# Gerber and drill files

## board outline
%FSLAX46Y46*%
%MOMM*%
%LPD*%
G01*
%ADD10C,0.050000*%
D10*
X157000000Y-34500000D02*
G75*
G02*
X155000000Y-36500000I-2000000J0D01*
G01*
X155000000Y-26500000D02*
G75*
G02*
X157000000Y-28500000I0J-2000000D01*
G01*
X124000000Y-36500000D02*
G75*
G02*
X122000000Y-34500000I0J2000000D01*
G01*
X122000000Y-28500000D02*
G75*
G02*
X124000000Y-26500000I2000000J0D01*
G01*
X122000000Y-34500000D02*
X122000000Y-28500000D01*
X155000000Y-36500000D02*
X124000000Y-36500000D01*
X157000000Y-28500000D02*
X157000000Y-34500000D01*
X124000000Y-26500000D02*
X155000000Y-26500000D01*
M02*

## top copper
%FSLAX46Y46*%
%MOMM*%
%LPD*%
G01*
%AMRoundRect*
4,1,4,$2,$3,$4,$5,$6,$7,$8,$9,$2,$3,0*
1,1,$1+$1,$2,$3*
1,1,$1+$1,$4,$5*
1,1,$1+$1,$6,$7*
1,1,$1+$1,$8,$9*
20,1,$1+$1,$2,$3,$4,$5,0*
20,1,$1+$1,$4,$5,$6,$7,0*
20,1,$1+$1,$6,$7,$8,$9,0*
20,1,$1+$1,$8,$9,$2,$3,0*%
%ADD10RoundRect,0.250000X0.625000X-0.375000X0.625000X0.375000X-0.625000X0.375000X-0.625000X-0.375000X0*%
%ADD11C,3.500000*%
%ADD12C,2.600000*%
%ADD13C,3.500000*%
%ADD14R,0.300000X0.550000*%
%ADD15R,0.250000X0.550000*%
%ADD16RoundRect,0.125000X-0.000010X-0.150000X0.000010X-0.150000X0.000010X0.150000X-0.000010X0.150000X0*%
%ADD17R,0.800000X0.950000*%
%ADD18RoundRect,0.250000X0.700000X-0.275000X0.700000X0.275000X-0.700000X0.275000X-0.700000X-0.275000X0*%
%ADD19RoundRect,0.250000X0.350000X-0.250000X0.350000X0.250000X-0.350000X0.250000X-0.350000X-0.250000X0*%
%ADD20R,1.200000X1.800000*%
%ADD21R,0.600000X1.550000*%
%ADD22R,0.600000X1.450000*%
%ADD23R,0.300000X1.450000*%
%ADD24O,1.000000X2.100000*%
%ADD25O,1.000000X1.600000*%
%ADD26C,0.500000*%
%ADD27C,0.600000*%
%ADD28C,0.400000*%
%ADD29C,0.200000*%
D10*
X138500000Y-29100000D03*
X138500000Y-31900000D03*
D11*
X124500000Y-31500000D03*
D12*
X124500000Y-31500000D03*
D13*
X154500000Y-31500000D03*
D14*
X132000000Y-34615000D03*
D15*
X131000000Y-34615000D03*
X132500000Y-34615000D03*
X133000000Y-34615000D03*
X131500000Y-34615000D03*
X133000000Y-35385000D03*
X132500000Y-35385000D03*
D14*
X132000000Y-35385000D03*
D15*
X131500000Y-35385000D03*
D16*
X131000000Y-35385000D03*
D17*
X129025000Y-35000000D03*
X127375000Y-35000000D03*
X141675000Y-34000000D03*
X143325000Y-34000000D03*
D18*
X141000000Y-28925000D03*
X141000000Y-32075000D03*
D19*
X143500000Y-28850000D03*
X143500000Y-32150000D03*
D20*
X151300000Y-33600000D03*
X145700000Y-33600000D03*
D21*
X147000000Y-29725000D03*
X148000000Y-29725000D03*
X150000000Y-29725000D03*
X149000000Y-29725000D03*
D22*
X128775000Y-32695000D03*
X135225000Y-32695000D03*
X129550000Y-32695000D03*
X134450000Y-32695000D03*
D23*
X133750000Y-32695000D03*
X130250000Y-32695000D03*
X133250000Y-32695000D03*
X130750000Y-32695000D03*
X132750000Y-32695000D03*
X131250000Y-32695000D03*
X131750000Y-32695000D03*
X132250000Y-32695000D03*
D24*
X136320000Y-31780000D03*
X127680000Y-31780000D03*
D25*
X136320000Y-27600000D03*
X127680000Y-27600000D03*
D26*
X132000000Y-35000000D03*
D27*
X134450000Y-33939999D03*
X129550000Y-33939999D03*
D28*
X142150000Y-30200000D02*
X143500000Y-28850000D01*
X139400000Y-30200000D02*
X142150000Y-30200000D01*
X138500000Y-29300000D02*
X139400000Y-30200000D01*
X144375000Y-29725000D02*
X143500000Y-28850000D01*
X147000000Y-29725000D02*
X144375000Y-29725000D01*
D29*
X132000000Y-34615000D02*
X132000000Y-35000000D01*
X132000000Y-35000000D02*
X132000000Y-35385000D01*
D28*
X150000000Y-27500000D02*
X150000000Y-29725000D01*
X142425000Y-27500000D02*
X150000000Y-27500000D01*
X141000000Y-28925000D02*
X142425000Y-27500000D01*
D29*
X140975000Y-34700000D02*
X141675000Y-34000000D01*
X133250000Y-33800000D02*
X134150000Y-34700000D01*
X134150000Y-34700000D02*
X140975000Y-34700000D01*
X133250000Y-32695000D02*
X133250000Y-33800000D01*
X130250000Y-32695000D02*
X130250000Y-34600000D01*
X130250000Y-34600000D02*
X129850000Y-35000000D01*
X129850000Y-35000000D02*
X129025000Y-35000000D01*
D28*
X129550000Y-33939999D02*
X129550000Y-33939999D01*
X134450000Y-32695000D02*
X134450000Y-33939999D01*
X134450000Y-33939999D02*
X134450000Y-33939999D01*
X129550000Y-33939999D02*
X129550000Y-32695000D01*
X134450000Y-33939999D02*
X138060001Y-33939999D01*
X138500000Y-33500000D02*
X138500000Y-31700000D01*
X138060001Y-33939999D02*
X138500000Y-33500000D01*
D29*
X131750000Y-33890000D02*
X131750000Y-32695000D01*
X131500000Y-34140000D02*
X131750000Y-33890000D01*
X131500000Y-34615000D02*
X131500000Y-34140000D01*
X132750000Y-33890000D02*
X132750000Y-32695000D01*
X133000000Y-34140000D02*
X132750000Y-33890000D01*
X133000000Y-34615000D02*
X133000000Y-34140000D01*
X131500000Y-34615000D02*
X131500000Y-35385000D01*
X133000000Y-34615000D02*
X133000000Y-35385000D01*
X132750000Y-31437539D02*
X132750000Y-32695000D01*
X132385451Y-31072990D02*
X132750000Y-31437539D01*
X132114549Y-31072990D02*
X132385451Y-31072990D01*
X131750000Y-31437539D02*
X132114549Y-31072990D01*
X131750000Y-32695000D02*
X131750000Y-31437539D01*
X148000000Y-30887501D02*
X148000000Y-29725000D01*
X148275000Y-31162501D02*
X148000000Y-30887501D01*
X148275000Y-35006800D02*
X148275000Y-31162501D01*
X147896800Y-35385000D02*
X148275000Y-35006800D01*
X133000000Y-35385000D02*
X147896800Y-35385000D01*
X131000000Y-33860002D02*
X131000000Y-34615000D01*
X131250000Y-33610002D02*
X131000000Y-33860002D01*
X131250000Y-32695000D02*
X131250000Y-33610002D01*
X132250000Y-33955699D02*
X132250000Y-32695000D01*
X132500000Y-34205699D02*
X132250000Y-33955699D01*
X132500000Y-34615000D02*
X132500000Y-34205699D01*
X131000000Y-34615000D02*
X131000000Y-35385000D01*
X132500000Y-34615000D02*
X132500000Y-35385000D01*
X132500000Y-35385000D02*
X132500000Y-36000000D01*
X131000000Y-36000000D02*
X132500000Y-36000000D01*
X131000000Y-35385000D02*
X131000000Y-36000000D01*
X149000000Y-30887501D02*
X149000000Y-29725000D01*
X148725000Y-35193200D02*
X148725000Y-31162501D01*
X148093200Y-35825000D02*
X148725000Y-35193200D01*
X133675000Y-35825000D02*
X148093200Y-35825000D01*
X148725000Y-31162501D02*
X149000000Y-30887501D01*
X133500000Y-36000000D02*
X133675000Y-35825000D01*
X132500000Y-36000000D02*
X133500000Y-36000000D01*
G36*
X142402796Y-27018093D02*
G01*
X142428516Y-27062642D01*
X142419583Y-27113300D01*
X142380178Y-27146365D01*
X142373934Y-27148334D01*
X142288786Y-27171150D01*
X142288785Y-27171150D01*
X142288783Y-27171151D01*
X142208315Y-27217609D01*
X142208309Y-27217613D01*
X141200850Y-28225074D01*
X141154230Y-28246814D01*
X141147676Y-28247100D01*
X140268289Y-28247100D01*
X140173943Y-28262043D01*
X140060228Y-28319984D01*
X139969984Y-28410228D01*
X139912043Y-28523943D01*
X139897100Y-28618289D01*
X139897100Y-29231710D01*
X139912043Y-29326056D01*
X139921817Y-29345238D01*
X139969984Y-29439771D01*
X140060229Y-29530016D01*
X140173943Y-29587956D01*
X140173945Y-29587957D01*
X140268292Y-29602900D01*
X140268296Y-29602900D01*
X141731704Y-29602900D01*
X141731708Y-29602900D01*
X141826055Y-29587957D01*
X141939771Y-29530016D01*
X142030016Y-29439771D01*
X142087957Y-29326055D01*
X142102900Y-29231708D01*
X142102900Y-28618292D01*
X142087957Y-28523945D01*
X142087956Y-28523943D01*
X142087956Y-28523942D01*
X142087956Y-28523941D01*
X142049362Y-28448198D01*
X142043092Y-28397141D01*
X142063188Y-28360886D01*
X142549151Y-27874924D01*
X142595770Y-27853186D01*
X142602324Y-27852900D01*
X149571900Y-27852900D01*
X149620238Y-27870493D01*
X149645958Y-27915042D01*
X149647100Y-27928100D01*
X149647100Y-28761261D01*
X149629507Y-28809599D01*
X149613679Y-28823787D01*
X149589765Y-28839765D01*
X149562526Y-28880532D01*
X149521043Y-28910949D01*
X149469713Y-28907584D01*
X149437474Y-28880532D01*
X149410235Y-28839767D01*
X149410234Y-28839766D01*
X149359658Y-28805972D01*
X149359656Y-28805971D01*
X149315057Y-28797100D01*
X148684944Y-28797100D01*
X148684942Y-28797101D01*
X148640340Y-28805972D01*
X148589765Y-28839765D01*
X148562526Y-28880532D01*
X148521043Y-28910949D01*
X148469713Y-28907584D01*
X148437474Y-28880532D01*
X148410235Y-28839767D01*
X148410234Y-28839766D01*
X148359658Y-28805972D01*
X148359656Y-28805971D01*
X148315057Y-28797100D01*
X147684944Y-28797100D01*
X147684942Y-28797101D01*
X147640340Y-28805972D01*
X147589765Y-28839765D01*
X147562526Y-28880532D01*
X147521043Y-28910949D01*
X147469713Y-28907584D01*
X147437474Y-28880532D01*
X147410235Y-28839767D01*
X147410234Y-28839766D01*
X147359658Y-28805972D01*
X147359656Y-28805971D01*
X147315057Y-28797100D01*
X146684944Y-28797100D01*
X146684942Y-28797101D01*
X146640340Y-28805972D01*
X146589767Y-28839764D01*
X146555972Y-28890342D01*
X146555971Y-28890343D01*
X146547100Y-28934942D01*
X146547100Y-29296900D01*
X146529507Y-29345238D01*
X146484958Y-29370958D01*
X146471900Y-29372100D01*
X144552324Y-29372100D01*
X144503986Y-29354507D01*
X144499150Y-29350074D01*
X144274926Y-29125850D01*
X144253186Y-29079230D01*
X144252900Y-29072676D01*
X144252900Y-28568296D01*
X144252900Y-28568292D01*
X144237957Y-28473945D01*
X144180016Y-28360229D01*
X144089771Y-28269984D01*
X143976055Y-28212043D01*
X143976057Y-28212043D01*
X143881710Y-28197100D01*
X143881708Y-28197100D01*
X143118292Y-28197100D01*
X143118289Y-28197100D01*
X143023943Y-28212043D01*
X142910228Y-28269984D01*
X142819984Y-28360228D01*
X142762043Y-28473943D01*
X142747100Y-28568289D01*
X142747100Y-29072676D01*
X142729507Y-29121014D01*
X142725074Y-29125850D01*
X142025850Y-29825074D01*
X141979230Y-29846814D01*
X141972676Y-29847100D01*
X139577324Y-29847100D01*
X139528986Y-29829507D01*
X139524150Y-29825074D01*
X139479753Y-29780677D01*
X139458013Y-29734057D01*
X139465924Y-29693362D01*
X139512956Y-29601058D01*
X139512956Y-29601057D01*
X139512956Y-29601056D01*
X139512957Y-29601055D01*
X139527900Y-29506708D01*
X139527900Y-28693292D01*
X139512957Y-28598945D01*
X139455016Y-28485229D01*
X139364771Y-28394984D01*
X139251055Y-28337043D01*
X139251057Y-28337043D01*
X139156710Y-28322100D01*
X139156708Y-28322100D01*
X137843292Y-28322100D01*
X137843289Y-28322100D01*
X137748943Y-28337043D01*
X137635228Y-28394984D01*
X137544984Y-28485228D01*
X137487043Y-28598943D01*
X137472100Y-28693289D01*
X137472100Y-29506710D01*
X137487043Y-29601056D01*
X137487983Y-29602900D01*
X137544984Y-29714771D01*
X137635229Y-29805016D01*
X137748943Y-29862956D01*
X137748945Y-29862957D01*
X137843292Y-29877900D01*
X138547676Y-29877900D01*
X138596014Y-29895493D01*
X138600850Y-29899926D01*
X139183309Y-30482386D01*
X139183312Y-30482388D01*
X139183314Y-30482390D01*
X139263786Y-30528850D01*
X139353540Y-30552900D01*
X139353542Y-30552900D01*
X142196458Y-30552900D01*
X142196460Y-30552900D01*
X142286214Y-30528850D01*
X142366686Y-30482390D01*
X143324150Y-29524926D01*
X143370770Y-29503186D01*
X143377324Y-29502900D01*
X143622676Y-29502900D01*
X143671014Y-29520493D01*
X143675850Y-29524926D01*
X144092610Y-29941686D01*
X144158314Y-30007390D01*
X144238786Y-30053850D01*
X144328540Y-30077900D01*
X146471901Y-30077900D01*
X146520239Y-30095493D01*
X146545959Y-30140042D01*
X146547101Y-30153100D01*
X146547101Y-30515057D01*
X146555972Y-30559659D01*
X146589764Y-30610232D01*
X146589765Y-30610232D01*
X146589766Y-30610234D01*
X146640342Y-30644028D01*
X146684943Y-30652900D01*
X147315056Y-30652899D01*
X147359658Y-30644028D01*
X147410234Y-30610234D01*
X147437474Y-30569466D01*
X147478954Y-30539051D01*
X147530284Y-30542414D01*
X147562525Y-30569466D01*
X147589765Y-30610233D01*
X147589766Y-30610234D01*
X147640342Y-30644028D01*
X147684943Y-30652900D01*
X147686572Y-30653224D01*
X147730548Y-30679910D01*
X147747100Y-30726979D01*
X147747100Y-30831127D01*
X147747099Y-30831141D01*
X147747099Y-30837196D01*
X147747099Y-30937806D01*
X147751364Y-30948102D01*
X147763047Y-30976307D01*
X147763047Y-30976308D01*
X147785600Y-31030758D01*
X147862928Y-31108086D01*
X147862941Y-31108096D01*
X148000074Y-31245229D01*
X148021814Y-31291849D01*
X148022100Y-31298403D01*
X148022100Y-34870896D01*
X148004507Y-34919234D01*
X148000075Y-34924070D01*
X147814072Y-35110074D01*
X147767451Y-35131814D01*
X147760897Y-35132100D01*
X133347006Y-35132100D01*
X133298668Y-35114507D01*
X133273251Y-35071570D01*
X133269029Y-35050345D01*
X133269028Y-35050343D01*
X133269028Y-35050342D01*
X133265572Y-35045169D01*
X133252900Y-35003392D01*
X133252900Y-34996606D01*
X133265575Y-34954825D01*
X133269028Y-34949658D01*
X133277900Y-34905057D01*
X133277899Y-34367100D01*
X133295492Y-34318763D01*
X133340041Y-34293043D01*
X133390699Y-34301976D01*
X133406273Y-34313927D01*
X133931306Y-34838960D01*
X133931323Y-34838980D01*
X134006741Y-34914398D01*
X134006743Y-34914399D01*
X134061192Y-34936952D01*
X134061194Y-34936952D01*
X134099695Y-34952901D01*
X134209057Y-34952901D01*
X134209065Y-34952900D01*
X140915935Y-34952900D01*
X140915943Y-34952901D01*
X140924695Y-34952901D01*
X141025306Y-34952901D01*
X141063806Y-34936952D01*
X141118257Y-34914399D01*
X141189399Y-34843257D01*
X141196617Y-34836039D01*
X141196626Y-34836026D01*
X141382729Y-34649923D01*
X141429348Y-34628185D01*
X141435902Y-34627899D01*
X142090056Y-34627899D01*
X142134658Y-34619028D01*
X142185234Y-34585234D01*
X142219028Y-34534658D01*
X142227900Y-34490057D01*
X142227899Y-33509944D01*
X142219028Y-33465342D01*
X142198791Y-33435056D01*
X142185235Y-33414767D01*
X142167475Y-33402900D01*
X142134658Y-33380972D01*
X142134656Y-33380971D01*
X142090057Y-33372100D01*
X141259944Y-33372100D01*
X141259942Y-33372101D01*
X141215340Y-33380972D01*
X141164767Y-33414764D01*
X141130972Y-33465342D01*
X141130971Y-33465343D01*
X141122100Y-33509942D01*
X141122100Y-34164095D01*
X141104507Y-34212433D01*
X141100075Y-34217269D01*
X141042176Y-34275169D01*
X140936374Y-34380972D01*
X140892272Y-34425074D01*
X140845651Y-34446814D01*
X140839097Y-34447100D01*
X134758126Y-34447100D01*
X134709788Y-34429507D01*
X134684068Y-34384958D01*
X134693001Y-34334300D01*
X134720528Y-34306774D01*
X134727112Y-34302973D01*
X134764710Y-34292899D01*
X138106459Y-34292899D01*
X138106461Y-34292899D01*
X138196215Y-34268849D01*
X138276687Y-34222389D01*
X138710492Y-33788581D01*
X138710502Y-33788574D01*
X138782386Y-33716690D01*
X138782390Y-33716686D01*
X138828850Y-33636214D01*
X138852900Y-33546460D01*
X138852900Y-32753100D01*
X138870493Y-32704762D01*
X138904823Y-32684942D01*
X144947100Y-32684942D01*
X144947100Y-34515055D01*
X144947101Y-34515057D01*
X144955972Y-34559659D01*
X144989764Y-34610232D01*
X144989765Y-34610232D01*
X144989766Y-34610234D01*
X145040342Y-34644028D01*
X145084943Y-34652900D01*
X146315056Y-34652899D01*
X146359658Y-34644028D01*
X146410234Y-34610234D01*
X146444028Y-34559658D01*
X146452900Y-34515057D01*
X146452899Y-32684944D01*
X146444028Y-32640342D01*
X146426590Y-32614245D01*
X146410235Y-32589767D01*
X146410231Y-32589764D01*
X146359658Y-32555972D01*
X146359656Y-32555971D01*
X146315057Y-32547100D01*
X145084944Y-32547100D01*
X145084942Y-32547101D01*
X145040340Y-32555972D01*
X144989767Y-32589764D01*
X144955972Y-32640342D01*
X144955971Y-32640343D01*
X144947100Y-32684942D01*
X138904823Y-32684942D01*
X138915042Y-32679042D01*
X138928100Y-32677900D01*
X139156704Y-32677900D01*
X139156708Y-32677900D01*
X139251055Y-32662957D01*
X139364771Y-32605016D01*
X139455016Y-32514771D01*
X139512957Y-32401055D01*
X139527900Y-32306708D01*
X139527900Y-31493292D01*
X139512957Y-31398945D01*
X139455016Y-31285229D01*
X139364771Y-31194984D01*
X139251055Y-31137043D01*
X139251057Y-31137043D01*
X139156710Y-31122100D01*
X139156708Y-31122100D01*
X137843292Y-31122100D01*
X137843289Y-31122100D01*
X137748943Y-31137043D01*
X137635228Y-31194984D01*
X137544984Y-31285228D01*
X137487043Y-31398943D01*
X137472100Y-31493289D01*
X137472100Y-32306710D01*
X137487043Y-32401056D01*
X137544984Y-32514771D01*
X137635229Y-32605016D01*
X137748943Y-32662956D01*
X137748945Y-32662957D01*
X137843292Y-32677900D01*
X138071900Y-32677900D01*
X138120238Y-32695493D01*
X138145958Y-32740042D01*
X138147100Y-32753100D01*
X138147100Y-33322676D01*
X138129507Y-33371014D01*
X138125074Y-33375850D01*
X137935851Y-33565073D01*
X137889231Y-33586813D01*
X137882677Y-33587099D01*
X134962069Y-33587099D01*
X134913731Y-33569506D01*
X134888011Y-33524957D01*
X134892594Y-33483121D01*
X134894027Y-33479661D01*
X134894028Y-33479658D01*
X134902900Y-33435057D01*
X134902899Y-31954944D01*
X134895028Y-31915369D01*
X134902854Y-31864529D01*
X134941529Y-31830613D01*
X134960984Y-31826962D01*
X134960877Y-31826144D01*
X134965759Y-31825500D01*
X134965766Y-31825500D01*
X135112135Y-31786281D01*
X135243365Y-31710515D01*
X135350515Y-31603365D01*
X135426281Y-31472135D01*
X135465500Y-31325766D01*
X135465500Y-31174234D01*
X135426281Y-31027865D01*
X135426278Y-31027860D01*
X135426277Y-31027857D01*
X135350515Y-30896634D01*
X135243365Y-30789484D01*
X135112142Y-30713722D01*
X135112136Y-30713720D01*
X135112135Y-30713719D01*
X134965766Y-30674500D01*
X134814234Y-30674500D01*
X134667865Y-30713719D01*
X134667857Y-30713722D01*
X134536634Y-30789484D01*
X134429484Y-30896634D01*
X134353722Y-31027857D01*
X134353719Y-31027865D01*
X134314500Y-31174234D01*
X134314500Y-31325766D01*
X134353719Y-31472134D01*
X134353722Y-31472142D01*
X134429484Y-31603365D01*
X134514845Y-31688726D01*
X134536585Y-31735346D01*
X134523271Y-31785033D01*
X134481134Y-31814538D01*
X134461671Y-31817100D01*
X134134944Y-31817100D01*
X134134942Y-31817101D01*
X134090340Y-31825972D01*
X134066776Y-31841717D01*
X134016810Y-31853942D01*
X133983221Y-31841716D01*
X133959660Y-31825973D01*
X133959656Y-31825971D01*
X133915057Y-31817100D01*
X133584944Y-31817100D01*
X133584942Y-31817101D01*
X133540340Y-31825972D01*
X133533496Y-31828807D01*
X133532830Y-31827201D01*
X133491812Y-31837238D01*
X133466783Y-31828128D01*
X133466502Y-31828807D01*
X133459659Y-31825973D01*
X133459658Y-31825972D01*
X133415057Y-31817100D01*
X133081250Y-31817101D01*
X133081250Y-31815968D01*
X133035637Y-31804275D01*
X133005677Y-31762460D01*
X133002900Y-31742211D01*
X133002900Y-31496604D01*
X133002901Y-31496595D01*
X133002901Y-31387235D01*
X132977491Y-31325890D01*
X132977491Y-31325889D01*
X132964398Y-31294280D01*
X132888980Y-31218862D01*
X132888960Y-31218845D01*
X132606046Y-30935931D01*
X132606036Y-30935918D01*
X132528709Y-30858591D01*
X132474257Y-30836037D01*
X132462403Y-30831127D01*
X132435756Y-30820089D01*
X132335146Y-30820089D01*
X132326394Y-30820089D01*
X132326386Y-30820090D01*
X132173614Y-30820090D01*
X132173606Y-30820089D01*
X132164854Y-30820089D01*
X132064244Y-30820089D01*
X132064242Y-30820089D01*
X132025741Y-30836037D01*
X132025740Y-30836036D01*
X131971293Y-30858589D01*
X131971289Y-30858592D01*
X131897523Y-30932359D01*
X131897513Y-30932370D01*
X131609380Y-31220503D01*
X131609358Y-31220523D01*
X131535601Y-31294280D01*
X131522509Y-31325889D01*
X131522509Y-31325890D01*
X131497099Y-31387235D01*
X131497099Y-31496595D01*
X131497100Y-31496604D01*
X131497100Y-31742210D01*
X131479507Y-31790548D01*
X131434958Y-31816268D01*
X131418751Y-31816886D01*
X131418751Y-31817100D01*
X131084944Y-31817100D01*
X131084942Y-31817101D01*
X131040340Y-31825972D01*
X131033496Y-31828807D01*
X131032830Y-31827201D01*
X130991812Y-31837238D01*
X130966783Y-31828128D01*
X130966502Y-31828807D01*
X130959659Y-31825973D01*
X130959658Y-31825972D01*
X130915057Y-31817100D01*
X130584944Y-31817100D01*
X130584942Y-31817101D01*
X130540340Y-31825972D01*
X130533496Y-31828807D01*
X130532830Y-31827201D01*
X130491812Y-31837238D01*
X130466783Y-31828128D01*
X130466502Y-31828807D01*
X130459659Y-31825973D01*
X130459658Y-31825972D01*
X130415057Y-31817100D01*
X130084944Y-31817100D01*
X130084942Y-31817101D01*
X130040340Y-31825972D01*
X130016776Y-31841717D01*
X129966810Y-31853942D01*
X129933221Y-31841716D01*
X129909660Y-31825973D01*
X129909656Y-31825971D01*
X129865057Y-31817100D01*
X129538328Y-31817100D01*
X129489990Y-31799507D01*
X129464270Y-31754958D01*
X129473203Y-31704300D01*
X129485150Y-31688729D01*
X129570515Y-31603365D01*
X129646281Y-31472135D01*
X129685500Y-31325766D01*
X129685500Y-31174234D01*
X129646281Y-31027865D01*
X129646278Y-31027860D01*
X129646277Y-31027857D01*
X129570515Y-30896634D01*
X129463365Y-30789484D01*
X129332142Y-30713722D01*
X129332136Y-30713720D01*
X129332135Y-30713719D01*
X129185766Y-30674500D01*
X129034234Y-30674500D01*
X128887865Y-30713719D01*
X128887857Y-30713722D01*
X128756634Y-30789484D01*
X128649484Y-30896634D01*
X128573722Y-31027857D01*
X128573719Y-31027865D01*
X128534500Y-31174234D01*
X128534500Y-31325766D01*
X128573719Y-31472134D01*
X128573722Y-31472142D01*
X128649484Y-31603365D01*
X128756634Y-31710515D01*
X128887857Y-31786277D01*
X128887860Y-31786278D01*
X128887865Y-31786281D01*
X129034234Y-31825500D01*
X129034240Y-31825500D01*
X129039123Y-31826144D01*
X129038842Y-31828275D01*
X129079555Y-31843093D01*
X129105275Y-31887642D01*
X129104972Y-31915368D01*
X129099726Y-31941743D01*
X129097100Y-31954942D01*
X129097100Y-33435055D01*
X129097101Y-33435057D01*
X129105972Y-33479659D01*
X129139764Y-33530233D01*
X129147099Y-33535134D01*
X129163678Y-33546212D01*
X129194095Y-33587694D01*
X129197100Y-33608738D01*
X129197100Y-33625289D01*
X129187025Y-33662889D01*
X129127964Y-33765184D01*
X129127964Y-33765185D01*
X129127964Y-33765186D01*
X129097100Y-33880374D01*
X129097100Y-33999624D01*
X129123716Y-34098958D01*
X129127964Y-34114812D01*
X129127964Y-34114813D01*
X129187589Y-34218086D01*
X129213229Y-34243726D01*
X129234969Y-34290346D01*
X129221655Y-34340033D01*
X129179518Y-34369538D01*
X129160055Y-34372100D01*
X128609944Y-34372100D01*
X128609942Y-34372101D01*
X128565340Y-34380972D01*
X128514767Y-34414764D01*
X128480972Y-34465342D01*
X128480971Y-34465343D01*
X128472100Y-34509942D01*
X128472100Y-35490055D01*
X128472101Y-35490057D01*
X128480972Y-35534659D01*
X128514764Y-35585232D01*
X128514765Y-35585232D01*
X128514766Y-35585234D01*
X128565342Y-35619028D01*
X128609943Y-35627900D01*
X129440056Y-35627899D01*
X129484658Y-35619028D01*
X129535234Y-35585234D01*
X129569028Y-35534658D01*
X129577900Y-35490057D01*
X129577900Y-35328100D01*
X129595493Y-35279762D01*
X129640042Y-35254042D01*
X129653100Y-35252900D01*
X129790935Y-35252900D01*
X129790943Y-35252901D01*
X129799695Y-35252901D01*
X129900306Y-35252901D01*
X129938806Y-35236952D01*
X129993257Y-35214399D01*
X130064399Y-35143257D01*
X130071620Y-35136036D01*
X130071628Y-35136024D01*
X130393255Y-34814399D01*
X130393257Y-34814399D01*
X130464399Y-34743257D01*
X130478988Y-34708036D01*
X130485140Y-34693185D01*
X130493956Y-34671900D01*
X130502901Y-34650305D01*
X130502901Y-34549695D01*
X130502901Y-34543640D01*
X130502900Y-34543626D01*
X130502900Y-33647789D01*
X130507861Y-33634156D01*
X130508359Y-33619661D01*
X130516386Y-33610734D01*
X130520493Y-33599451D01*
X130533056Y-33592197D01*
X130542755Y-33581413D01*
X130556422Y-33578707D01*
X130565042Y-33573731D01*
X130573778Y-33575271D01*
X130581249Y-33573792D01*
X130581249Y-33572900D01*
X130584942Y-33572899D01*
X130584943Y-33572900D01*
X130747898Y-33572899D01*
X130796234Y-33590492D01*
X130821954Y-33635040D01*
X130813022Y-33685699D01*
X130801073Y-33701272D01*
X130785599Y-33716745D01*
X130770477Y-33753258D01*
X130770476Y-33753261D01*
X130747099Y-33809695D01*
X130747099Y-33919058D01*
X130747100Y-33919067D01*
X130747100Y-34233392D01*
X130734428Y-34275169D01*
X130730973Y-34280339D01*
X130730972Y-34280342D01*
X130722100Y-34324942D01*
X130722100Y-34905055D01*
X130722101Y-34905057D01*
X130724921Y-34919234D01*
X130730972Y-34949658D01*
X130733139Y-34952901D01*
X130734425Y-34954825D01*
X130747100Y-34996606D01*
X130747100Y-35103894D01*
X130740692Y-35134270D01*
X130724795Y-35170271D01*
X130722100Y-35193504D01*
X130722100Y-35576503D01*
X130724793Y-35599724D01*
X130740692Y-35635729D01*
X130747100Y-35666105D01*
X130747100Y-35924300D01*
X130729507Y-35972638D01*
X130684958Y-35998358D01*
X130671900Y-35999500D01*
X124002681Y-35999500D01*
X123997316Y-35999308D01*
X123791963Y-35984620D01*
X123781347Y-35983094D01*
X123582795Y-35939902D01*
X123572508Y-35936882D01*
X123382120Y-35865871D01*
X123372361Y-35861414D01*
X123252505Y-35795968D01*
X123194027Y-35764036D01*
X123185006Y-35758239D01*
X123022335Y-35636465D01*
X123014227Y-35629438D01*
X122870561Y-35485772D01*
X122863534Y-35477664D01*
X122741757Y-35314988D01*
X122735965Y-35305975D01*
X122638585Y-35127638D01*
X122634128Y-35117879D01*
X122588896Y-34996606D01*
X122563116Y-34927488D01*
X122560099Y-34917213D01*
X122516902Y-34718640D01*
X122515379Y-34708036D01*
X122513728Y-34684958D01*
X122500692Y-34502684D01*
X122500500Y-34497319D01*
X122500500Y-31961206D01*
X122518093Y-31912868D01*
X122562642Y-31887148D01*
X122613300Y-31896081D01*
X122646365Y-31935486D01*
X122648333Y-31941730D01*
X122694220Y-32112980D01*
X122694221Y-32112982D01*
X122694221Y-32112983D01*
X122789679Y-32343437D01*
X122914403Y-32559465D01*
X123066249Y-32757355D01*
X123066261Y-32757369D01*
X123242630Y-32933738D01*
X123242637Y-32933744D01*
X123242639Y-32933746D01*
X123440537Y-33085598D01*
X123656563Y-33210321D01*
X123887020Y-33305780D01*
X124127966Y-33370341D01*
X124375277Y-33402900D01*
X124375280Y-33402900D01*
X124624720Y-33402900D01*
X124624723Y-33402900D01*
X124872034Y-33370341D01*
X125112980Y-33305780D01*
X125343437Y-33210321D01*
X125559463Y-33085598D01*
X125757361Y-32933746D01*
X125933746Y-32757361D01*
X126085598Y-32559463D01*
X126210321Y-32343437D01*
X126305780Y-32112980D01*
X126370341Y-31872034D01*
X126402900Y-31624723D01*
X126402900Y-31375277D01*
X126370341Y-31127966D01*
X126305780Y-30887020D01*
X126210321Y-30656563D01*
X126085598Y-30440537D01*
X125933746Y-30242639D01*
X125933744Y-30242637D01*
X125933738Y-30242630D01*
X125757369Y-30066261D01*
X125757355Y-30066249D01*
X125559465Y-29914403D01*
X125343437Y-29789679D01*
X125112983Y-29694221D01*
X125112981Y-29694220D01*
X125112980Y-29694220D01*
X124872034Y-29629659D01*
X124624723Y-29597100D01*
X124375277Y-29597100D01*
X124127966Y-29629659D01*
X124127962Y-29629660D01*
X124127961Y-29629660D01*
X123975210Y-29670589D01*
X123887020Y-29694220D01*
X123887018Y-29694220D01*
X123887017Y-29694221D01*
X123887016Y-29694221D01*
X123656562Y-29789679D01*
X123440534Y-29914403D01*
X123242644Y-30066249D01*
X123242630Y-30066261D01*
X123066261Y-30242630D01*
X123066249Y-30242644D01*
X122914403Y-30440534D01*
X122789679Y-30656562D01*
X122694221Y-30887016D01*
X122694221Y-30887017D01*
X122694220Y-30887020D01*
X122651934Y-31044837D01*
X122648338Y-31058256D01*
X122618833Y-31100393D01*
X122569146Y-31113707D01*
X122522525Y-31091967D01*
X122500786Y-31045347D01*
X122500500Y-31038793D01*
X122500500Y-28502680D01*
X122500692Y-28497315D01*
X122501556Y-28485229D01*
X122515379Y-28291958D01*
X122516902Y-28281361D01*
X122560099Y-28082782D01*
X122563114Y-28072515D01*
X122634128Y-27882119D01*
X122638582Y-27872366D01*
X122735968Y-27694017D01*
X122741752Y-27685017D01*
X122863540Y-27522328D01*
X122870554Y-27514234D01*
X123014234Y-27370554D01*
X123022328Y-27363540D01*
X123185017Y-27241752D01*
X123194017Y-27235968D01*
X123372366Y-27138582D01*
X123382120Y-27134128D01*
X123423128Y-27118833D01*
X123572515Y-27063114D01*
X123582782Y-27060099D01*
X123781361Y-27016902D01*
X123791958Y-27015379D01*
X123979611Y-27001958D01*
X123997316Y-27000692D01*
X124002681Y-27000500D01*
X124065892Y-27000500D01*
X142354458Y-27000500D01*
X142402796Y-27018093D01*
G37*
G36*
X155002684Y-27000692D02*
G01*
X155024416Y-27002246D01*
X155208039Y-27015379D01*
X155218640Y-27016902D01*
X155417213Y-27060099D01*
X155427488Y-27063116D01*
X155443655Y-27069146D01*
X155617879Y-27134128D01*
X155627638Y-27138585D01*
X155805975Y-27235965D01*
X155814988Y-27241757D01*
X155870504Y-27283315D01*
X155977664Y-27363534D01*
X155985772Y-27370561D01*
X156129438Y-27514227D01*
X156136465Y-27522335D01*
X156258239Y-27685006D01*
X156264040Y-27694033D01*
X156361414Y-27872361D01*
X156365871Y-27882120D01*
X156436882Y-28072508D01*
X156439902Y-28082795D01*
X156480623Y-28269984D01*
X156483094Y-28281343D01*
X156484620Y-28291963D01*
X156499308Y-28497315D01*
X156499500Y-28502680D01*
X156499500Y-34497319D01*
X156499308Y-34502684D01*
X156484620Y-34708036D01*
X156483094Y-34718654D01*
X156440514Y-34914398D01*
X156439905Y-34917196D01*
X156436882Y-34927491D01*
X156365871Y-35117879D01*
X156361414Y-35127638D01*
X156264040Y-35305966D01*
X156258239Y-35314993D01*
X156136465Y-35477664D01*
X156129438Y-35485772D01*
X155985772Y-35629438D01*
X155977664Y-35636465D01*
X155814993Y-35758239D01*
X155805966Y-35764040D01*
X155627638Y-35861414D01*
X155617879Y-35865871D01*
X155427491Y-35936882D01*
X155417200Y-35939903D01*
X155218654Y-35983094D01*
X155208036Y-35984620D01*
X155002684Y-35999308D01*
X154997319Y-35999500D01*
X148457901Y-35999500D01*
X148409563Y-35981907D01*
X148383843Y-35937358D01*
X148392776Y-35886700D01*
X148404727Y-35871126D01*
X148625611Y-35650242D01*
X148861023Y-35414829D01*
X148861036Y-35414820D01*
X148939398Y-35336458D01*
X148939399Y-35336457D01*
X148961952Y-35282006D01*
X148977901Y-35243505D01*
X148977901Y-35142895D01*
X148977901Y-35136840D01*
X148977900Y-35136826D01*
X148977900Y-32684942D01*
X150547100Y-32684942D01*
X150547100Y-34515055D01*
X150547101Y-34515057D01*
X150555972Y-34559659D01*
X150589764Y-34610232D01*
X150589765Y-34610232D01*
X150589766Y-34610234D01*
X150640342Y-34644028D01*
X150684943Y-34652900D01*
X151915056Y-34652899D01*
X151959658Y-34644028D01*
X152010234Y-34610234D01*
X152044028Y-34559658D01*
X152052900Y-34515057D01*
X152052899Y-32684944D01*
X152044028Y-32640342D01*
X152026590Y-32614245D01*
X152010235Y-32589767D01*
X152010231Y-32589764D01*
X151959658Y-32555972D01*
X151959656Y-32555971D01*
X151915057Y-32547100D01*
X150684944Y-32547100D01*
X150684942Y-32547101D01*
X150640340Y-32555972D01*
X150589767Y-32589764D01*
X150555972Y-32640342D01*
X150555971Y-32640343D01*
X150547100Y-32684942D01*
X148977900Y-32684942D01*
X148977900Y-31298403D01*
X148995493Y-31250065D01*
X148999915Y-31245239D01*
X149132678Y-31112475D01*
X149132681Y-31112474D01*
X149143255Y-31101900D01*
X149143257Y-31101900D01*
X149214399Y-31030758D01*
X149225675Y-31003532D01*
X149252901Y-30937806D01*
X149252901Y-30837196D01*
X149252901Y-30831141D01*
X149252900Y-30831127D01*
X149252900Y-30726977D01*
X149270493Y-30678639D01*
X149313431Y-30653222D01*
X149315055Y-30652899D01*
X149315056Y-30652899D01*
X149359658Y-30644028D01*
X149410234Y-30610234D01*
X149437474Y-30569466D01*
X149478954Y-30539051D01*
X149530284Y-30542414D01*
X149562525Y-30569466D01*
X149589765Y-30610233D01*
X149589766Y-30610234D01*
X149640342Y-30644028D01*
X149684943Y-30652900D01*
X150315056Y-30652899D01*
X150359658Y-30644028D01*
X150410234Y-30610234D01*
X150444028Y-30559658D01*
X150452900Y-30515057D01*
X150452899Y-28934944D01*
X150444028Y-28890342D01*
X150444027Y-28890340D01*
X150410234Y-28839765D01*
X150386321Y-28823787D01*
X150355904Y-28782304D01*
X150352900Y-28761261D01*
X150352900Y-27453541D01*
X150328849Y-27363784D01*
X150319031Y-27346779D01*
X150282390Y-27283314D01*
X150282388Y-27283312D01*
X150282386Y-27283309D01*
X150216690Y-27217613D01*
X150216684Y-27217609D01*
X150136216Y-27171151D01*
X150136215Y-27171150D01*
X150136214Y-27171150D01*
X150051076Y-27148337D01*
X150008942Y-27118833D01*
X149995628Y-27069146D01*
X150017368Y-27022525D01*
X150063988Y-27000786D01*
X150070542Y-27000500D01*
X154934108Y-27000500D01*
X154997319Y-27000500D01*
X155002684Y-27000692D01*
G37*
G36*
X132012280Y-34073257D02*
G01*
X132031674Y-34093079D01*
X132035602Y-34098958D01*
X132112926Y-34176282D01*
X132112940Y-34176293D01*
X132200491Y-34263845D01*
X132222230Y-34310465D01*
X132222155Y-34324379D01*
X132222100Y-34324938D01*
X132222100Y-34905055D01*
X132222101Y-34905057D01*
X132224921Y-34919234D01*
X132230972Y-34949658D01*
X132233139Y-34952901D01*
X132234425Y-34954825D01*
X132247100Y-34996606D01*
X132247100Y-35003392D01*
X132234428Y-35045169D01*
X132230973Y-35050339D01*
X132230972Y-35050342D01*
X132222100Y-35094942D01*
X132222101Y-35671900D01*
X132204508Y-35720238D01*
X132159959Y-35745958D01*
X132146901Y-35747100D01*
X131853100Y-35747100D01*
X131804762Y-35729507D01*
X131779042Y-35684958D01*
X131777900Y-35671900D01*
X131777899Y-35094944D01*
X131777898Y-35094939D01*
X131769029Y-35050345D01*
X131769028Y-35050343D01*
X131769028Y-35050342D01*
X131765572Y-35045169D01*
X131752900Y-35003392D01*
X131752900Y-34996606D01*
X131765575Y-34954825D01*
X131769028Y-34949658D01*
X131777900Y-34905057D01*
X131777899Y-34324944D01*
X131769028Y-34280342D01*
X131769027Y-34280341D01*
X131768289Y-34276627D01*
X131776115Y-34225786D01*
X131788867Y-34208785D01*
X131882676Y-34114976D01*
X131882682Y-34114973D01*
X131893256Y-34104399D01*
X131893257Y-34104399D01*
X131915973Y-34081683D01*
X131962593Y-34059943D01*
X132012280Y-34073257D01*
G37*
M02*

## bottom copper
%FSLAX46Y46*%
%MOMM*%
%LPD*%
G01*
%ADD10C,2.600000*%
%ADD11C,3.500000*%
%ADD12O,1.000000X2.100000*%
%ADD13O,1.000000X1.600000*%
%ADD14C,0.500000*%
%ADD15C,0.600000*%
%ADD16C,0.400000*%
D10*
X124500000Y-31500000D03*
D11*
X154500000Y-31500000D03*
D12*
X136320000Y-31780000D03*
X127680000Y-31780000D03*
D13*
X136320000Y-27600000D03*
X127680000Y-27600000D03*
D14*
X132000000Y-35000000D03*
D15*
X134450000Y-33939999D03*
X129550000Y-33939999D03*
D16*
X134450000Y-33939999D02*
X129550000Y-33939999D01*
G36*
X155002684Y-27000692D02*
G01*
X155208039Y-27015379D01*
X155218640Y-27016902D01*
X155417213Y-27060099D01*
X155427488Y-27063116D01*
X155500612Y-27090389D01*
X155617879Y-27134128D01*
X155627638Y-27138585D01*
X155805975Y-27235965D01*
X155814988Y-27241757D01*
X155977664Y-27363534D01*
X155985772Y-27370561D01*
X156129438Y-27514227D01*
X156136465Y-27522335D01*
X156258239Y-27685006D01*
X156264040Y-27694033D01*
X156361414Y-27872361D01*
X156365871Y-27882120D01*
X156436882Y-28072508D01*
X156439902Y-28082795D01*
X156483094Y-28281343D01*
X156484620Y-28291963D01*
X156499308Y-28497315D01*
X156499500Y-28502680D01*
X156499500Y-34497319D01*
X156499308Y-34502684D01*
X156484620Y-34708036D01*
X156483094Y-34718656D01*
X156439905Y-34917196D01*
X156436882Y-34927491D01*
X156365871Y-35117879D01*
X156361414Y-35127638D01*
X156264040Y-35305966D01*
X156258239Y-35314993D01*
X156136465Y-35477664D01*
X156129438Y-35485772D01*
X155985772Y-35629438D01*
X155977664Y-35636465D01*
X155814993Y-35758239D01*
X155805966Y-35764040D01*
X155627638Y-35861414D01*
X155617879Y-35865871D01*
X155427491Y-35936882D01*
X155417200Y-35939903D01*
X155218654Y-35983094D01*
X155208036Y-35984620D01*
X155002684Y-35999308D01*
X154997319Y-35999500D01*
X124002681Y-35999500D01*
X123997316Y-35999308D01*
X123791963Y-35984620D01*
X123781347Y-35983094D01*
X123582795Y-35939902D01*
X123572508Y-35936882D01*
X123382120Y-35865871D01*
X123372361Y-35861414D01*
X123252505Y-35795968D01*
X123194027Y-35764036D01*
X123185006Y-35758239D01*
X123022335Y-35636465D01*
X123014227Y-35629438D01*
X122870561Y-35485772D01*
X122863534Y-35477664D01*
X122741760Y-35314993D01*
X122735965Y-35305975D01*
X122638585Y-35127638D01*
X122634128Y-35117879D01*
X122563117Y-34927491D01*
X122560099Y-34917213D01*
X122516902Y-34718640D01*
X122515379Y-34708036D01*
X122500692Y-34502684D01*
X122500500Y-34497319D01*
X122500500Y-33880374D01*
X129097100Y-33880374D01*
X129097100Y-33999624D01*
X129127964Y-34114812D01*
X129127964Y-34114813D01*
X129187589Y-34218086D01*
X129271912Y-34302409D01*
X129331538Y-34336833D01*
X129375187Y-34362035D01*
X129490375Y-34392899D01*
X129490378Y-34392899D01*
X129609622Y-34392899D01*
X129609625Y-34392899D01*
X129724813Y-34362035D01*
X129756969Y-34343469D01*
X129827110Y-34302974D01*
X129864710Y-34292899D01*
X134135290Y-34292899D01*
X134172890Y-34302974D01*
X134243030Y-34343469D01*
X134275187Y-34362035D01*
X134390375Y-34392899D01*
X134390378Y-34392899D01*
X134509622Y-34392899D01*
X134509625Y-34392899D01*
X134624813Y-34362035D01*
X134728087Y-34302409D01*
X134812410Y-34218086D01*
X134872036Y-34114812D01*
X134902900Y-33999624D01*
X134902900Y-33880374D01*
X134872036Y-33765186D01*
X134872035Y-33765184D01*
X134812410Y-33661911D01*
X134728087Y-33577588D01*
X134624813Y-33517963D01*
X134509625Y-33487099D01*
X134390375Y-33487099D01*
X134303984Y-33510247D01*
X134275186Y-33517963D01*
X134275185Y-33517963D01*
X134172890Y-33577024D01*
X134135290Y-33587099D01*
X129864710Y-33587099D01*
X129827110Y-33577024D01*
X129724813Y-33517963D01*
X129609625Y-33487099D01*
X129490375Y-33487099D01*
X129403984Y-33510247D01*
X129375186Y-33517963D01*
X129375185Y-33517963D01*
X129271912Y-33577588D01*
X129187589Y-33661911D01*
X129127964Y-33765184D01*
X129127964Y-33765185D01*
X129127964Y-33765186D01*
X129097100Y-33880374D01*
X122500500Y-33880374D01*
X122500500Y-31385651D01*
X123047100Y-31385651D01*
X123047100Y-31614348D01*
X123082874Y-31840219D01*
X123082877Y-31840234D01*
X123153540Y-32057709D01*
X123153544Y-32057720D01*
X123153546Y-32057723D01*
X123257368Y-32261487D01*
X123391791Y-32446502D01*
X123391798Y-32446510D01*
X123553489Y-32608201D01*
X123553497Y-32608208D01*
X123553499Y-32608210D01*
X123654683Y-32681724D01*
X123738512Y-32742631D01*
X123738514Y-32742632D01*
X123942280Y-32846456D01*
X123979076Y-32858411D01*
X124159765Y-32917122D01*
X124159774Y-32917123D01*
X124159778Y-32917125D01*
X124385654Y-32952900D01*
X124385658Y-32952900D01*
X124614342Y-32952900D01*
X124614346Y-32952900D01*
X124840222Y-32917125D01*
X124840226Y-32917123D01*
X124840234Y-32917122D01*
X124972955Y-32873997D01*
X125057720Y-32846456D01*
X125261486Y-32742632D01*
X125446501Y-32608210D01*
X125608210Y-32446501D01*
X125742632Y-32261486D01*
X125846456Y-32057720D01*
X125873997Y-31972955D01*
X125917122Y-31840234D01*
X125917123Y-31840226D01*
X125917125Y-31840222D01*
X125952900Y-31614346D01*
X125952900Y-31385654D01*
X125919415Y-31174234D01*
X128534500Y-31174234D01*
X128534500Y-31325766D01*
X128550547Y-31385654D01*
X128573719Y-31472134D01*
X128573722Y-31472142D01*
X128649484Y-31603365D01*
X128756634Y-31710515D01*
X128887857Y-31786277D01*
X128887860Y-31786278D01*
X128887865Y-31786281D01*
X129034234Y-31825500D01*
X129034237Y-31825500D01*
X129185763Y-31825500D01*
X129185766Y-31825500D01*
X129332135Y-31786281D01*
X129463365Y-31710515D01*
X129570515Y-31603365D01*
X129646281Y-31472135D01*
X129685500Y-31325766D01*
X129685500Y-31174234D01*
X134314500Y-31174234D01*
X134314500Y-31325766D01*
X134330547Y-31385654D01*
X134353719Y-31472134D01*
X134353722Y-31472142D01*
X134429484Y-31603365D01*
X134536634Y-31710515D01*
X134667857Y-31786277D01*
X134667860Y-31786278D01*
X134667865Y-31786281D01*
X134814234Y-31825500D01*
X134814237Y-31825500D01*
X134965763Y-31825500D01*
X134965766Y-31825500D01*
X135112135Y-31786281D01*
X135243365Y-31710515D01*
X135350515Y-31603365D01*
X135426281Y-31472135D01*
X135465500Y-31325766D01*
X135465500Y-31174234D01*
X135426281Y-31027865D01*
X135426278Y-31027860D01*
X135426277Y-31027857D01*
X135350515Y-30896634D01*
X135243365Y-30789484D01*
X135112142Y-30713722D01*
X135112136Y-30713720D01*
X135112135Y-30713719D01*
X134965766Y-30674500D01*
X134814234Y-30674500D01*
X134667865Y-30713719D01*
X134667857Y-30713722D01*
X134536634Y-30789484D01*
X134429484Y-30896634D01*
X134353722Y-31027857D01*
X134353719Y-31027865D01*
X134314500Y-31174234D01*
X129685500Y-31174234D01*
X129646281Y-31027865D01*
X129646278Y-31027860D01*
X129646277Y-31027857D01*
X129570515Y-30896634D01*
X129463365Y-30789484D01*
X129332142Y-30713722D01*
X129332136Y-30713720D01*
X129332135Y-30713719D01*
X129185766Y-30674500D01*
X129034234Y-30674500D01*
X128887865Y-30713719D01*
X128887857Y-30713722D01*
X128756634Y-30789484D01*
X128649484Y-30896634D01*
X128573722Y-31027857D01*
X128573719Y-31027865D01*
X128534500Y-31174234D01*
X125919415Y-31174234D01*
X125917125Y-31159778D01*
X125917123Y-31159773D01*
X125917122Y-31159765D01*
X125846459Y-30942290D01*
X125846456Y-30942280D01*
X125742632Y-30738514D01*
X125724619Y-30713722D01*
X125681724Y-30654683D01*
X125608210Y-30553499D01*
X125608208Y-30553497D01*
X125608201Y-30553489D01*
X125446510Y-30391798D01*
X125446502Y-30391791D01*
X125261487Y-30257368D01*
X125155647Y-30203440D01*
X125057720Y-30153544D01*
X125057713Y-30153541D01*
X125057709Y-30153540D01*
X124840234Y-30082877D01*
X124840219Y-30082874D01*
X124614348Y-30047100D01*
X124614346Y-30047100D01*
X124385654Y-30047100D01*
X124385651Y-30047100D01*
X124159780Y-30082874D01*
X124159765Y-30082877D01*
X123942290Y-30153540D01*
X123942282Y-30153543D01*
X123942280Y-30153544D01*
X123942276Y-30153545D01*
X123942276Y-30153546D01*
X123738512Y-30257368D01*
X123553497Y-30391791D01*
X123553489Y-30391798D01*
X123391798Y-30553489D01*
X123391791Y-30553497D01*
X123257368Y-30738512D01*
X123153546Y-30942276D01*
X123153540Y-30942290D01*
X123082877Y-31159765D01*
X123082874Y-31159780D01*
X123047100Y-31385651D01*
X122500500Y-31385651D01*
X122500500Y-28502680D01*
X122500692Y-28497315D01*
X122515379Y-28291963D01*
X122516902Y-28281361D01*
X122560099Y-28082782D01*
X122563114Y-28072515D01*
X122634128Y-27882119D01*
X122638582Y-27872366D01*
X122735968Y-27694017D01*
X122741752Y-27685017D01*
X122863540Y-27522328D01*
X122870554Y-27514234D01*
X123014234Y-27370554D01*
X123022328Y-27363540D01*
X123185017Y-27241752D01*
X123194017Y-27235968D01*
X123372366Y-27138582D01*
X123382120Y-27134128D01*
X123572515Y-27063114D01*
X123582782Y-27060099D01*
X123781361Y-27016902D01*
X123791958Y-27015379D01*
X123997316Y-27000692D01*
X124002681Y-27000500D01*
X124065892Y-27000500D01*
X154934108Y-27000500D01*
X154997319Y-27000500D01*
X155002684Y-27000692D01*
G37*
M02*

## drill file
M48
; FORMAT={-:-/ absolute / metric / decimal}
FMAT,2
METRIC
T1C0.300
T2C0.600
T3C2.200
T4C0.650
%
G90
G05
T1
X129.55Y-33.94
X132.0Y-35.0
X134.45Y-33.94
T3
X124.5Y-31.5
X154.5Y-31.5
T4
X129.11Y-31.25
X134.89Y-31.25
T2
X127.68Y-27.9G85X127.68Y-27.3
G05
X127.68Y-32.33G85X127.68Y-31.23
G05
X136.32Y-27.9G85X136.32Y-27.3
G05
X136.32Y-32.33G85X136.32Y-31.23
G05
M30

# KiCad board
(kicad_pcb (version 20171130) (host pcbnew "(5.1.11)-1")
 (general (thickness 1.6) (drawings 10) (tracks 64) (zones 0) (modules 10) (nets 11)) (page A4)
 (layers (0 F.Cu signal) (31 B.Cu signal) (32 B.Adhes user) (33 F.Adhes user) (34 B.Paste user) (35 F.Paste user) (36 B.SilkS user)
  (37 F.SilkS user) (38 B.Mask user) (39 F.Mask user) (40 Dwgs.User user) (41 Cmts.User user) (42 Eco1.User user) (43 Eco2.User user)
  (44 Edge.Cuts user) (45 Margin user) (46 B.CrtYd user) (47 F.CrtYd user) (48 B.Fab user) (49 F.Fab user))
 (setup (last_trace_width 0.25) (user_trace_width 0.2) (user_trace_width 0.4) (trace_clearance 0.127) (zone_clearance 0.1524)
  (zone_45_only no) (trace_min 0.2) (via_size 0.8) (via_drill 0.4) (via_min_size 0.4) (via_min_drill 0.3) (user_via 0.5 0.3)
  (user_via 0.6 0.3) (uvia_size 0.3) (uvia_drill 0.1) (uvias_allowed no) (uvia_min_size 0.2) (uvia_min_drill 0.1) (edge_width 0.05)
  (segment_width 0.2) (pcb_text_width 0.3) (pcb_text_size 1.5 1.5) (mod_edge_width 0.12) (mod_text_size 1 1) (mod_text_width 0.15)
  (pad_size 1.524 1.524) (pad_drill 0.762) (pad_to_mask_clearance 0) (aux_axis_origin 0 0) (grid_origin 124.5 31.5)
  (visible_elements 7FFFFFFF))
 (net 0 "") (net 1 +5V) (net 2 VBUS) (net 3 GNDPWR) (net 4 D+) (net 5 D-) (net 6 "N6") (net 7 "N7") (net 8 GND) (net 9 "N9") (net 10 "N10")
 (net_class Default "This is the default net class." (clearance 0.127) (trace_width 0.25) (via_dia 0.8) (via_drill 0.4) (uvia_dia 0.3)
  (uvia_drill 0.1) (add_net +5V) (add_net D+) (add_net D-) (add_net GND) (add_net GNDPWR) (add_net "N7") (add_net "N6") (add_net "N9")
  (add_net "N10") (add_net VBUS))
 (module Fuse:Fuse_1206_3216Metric (layer F.Cu) (at 138.5 30.5 90)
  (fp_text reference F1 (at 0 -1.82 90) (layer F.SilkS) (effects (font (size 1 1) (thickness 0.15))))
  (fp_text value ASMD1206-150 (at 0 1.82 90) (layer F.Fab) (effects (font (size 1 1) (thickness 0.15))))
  (pad 2 smd roundrect (at 1.4 0 90) (size 1.25 1.75) (layers F.Cu F.Paste F.Mask) (roundrect_rratio 0.2) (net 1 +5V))
  (pad 1 smd roundrect (at -1.4 0 90) (size 1.25 1.75) (layers F.Cu F.Paste F.Mask) (roundrect_rratio 0.2) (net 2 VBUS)))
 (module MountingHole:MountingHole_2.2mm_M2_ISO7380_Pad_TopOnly (layer F.Cu) (at 124.5 31.5)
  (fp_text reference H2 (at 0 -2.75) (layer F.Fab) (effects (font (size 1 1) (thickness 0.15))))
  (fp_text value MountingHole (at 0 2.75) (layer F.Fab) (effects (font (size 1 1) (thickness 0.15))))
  (pad 1 connect circle (at 0 0) (size 3.5 3.5) (layers F.Cu F.Mask))
  (pad 1 thru_hole circle (at 0 0) (size 2.6 2.6) (drill 2.2) (layers *.Cu *.Mask)))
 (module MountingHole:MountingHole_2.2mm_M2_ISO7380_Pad (layer F.Cu) (at 154.5 31.5)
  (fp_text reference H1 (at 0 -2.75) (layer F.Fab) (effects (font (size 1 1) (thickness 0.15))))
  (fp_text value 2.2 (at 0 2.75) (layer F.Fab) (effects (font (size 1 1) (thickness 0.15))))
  (pad 1 thru_hole circle (at 0 0) (size 3.5 3.5) (drill 2.2) (layers *.Cu *.Mask) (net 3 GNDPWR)))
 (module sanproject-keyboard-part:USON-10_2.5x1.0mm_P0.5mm (layer F.Cu) (at 132 35 90)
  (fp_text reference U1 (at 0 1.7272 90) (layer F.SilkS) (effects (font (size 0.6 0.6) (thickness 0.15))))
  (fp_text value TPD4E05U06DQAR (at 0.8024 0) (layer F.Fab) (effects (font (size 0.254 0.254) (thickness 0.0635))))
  (pad 8 smd rect (at 0.385 0) (size 0.3 0.55) (layers F.Cu F.Paste F.Mask) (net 3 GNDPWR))
  (pad 10 smd rect (at 0.385 -1) (size 0.25 0.55) (layers F.Cu F.Paste F.Mask) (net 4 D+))
  (pad 7 smd rect (at 0.385 0.5) (size 0.25 0.55) (layers F.Cu F.Paste F.Mask) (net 4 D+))
  (pad 6 smd rect (at 0.385 1) (size 0.25 0.55) (layers F.Cu F.Paste F.Mask) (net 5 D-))
  (pad 9 smd rect (at 0.385 -0.5) (size 0.25 0.55) (layers F.Cu F.Paste F.Mask) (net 5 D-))
  (pad 5 smd rect (at -0.385 1) (size 0.25 0.55) (layers F.Cu F.Paste F.Mask) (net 5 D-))
  (pad 4 smd rect (at -0.385 0.5) (size 0.25 0.55) (layers F.Cu F.Paste F.Mask) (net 4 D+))
  (pad 3 smd rect (at -0.385 0) (size 0.3 0.55) (layers F.Cu F.Paste F.Mask) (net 3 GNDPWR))
  (pad 2 smd rect (at -0.385 -0.5) (size 0.25 0.55) (layers F.Cu F.Paste F.Mask) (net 5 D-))
  (pad 1 smd roundrect (at -0.385 -1) (size 0.25 0.55) (layers F.Cu F.Paste F.Mask) (roundrect_rratio 0.5) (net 4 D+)))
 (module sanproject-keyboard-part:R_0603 (layer F.Cu) (at 128.2 35)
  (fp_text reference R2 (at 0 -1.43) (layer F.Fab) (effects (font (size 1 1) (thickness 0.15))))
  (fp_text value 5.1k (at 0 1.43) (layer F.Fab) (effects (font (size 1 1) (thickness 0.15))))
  (pad 2 smd rect (at 0.825 0) (size 0.8 0.95) (layers F.Cu F.Paste F.Mask) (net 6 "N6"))
  (pad 1 smd rect (at -0.825 0) (size 0.8 0.95) (layers F.Cu F.Paste F.Mask) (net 3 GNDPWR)))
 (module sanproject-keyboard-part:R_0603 (layer F.Cu) (at 142.5 34 180)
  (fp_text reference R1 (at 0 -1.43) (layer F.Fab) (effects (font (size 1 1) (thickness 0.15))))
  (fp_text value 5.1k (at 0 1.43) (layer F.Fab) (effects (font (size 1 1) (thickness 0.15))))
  (pad 2 smd rect (at 0.825 0 180) (size 0.8 0.95) (layers F.Cu F.Paste F.Mask) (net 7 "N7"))
  (pad 1 smd rect (at -0.825 0 180) (size 0.8 0.95) (layers F.Cu F.Paste F.Mask) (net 3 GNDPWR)))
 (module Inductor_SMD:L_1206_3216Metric (layer F.Cu) (at 141 30.5 90)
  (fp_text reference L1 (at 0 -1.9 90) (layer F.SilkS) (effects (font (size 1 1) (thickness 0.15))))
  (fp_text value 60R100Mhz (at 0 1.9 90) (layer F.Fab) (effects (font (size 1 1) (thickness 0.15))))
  (pad 2 smd roundrect (at 1.575 0 90) (size 1.05 1.9) (layers F.Cu F.Paste F.Mask) (roundrect_rratio 0.238095) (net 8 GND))
  (pad 1 smd roundrect (at -1.575 0 90) (size 1.05 1.9) (layers F.Cu F.Paste F.Mask) (roundrect_rratio 0.238095) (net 3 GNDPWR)))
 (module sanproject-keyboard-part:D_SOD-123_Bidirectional (layer F.Cu) (at 143.5 30.5 90)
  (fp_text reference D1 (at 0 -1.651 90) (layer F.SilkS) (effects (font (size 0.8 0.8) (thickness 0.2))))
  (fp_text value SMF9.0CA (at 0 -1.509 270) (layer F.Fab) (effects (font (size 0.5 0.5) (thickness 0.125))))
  (pad 2 smd roundrect (at 1.65 0 90) (size 1 1.2) (layers F.Cu F.Paste F.Mask) (roundrect_rratio 0.25) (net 1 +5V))
  (pad 1 smd roundrect (at -1.65 0 90) (size 1 1.2) (layers F.Cu F.Paste F.Mask) (roundrect_rratio 0.25) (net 3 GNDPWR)))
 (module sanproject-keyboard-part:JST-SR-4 (layer F.Cu) (at 148.5 34.5)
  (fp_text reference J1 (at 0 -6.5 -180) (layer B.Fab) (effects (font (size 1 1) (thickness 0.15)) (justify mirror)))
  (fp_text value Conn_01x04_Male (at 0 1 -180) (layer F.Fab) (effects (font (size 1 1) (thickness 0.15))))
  (pad "" smd rect (at 2.8 -0.9) (size 1.2 1.8) (layers F.Cu F.Paste F.Mask))
  (pad "" smd rect (at -2.8 -0.9) (size 1.2 1.8) (layers F.Cu F.Paste F.Mask))
  (pad 1 smd rect (at -1.5 -4.775) (size 0.6 1.55) (layers F.Cu F.Paste F.Mask) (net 1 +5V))
  (pad 2 smd rect (at -0.5 -4.775) (size 0.6 1.55) (layers F.Cu F.Paste F.Mask) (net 5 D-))
  (pad 4 smd rect (at 1.5 -4.775) (size 0.6 1.55) (layers F.Cu F.Paste F.Mask) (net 8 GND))
  (pad 3 smd rect (at 0.5 -4.775) (size 0.6 1.55) (layers F.Cu F.Paste F.Mask) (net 4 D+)))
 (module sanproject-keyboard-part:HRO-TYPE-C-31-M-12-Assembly (layer F.Cu) (at 132 25 180)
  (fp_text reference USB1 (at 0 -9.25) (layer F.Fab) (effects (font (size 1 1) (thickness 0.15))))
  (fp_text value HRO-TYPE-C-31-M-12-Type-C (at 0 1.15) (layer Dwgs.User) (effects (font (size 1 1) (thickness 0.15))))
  (pad 12 smd rect (at 3.225 -7.695 180) (size 0.6 1.45) (layers F.Cu F.Paste F.Mask) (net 3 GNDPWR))
  (pad 1 smd rect (at -3.225 -7.695 180) (size 0.6 1.45) (layers F.Cu F.Paste F.Mask) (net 3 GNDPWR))
  (pad 11 smd rect (at 2.45 -7.695 180) (size 0.6 1.45) (layers F.Cu F.Paste F.Mask) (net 2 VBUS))
  (pad 2 smd rect (at -2.45 -7.695 180) (size 0.6 1.45) (layers F.Cu F.Paste F.Mask) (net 2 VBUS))
  (pad 3 smd rect (at -1.75 -7.695 180) (size 0.3 1.45) (layers F.Cu F.Paste F.Mask) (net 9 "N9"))
  (pad 10 smd rect (at 1.75 -7.695 180) (size 0.3 1.45) (layers F.Cu F.Paste F.Mask) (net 6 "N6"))
  (pad 4 smd rect (at -1.25 -7.695 180) (size 0.3 1.45) (layers F.Cu F.Paste F.Mask) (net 7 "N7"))
  (pad 9 smd rect (at 1.25 -7.695 180) (size 0.3 1.45) (layers F.Cu F.Paste F.Mask) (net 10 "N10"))
  (pad 5 smd rect (at -0.75 -7.695 180) (size 0.3 1.45) (layers F.Cu F.Paste F.Mask) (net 5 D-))
  (pad 8 smd rect (at 0.75 -7.695 180) (size 0.3 1.45) (layers F.Cu F.Paste F.Mask) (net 4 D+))
  (pad 7 smd rect (at 0.25 -7.695 180) (size 0.3 1.45) (layers F.Cu F.Paste F.Mask) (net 5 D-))
  (pad 6 smd rect (at -0.25 -7.695 180) (size 0.3 1.45) (layers F.Cu F.Paste F.Mask) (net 4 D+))
  (pad "" np_thru_hole circle (at 2.89 -6.25 180) (size 0.65 0.65) (drill 0.65) (layers *.Cu *.Mask))
  (pad "" np_thru_hole circle (at -2.89 -6.25 180) (size 0.65 0.65) (drill 0.65) (layers *.Cu *.Mask))
  (pad 13 thru_hole oval (at -4.32 -6.78 180) (size 1 2.1) (drill oval 0.6 1.7) (layers *.Cu *.Mask F.Paste) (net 3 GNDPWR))
  (pad 13 thru_hole oval (at 4.32 -6.78 180) (size 1 2.1) (drill oval 0.6 1.7) (layers *.Cu *.Mask F.Paste) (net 3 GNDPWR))
  (pad 13 thru_hole oval (at -4.32 -2.6 180) (size 1 1.6) (drill oval 0.6 1.2) (layers *.Cu *.Mask F.Paste) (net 3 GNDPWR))
  (pad 13 thru_hole oval (at 4.32 -2.6 180) (size 1 1.6) (drill oval 0.6 1.2) (layers *.Cu *.Mask F.Paste) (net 3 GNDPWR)))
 (gr_arc (start 155 34.5) (end 155 36.5) (angle -90) (layer Edge.Cuts) (width 0.05))
 (gr_arc (start 155 28.5) (end 157 28.5) (angle -90) (layer Edge.Cuts) (width 0.05))
 (gr_arc (start 124 34.5) (end 122 34.5) (angle -90) (layer Edge.Cuts) (width 0.05))
 (gr_arc (start 124 28.5) (end 124 26.5) (angle -90) (layer Edge.Cuts) (width 0.05))
 (gr_line (start 122 34.5) (end 122 28.5) (layer Edge.Cuts) (width 0.05))
 (gr_line (start 155 36.5) (end 124 36.5) (layer Edge.Cuts) (width 0.05))
 (gr_line (start 157 28.5) (end 157 34.5) (layer Edge.Cuts) (width 0.05))
 (gr_line (start 124 26.5) (end 155 26.5) (layer Edge.Cuts) (width 0.05))
 (segment (start 142.15 30.2) (end 143.5 28.85) (width 0.4) (layer F.Cu) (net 1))
 (segment (start 139.4 30.2) (end 142.15 30.2) (width 0.4) (layer F.Cu) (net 1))
 (segment (start 138.5 29.3) (end 139.4 30.2) (width 0.4) (layer F.Cu) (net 1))
 (segment (start 144.375 29.725) (end 143.5 28.85) (width 0.4) (layer F.Cu) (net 1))
 (segment (start 147 29.725) (end 144.375 29.725) (width 0.4) (layer F.Cu) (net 1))
 (via (at 132 35) (size 0.5) (drill 0.3) (layers F.Cu B.Cu) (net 3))
 (segment (start 132 34.615) (end 132 35) (width 0.2) (layer F.Cu) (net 3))
 (segment (start 132 35) (end 132 35.385) (width 0.2) (layer F.Cu) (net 3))
 (segment (start 150 27.5) (end 150 29.725) (width 0.4) (layer F.Cu) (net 8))
 (segment (start 142.425 27.5) (end 150 27.5) (width 0.4) (layer F.Cu) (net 8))
 (segment (start 141 28.925) (end 142.425 27.5) (width 0.4) (layer F.Cu) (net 8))
 (segment (start 140.975 34.7) (end 141.675 34) (width 0.2) (layer F.Cu) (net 7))
 (segment (start 133.25 33.8) (end 134.15 34.7) (width 0.2) (layer F.Cu) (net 7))
 (segment (start 134.15 34.7) (end 140.975 34.7) (width 0.2) (layer F.Cu) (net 7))
 (segment (start 133.25 32.695) (end 133.25 33.8) (width 0.2) (layer F.Cu) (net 7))
 (segment (start 130.25 32.695) (end 130.25 34.6) (width 0.2) (layer F.Cu) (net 6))
 (segment (start 130.25 34.6) (end 129.85 35) (width 0.2) (layer F.Cu) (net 6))
 (segment (start 129.85 35) (end 129.025 35) (width 0.2) (layer F.Cu) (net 6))
 (segment (start 129.55 33.939999) (end 129.55 33.939999) (width 0.4) (layer F.Cu) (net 2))
 (segment (start 134.45 32.695) (end 134.45 33.939999) (width 0.4) (layer F.Cu) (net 2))
 (segment (start 134.45 33.939999) (end 134.45 33.939999) (width 0.4) (layer F.Cu) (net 2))
 (via (at 134.45 33.939999) (size 0.6) (drill 0.3) (layers F.Cu B.Cu) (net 2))
 (segment (start 129.55 33.939999) (end 129.55 32.695) (width 0.4) (layer F.Cu) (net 2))
 (via (at 129.55 33.939999) (size 0.6) (drill 0.3) (layers F.Cu B.Cu) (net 2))
 (segment (start 134.45 33.939999) (end 129.55 33.939999) (width 0.4) (layer B.Cu) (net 2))
 (segment (start 134.45 33.939999) (end 138.060001 33.939999) (width 0.4) (layer F.Cu) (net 2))
 (segment (start 138.5 33.5) (end 138.5 31.7) (width 0.4) (layer F.Cu) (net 2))
 (segment (start 138.060001 33.939999) (end 138.5 33.5) (width 0.4) (layer F.Cu) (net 2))
 (segment (start 131.75 33.89) (end 131.75 32.695) (width 0.2) (layer F.Cu) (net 5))
 (segment (start 131.5 34.14) (end 131.75 33.89) (width 0.2) (layer F.Cu) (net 5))
 (segment (start 131.5 34.615) (end 131.5 34.14) (width 0.2) (layer F.Cu) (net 5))
 (segment (start 132.75 33.89) (end 132.75 32.695) (width 0.2) (layer F.Cu) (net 5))
 (segment (start 133 34.14) (end 132.75 33.89) (width 0.2) (layer F.Cu) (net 5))
 (segment (start 133 34.615) (end 133 34.14) (width 0.2) (layer F.Cu) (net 5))
 (segment (start 131.5 34.615) (end 131.5 35.385) (width 0.2) (layer F.Cu) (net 5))
 (segment (start 133 34.615) (end 133 35.385) (width 0.2) (layer F.Cu) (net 5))
 (segment (start 132.75 31.437539) (end 132.75 32.695) (width 0.2) (layer F.Cu) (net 5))
 (segment (start 132.385451 31.07299) (end 132.75 31.437539) (width 0.2) (layer F.Cu) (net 5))
 (segment (start 132.114549 31.07299) (end 132.385451 31.07299) (width 0.2) (layer F.Cu) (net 5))
 (segment (start 131.75 31.437539) (end 132.114549 31.07299) (width 0.2) (layer F.Cu) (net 5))
 (segment (start 131.75 32.695) (end 131.75 31.437539) (width 0.2) (layer F.Cu) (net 5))
 (segment (start 148 30.887501) (end 148 29.725) (width 0.2) (layer F.Cu) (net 5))
 (segment (start 148.275 31.162501) (end 148 30.887501) (width 0.2) (layer F.Cu) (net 5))
 (segment (start 148.275 35.0068) (end 148.275 31.162501) (width 0.2) (layer F.Cu) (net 5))
 (segment (start 147.8968 35.385) (end 148.275 35.0068) (width 0.2) (layer F.Cu) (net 5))
 (segment (start 133 35.385) (end 147.8968 35.385) (width 0.2) (layer F.Cu) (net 5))
 (segment (start 131 33.860002) (end 131 34.615) (width 0.2) (layer F.Cu) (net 4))
 (segment (start 131.25 33.610002) (end 131 33.860002) (width 0.2) (layer F.Cu) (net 4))
 (segment (start 131.25 32.695) (end 131.25 33.610002) (width 0.2) (layer F.Cu) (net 4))
 (segment (start 132.25 33.955699) (end 132.25 32.695) (width 0.2) (layer F.Cu) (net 4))
 (segment (start 132.5 34.205699) (end 132.25 33.955699) (width 0.2) (layer F.Cu) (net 4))
 (segment (start 132.5 34.615) (end 132.5 34.205699) (width 0.2) (layer F.Cu) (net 4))
 (segment (start 131 34.615) (end 131 35.385) (width 0.2) (layer F.Cu) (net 4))
 (segment (start 132.5 34.615) (end 132.5 35.385) (width 0.2) (layer F.Cu) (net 4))
 (segment (start 132.5 35.385) (end 132.5 36) (width 0.2) (layer F.Cu) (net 4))
 (segment (start 131 36) (end 132.5 36) (width 0.2) (layer F.Cu) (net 4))
 (segment (start 131 35.385) (end 131 36) (width 0.2) (layer F.Cu) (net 4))
 (segment (start 149 30.887501) (end 149 29.725) (width 0.2) (layer F.Cu) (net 4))
 (segment (start 148.725 35.1932) (end 148.725 31.162501) (width 0.2) (layer F.Cu) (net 4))
 (segment (start 148.0932 35.825) (end 148.725 35.1932) (width 0.2) (layer F.Cu) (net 4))
 (segment (start 133.675 35.825) (end 148.0932 35.825) (width 0.2) (layer F.Cu) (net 4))
 (segment (start 148.725 31.162501) (end 149 30.887501) (width 0.2) (layer F.Cu) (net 4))
 (segment (start 133.5 36) (end 133.675 35.825) (width 0.2) (layer F.Cu) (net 4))
 (segment (start 132.5 36) (end 133.5 36) (width 0.2) (layer F.Cu) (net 4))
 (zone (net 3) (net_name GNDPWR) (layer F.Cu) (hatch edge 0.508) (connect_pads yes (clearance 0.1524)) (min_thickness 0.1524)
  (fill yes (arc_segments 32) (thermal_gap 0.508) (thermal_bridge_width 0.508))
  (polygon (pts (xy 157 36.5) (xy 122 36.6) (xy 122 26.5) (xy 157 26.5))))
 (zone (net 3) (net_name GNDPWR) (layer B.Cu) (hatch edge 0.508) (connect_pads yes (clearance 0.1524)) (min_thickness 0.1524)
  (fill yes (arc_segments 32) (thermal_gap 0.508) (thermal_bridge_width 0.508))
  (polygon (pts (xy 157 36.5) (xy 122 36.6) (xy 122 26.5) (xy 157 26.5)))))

